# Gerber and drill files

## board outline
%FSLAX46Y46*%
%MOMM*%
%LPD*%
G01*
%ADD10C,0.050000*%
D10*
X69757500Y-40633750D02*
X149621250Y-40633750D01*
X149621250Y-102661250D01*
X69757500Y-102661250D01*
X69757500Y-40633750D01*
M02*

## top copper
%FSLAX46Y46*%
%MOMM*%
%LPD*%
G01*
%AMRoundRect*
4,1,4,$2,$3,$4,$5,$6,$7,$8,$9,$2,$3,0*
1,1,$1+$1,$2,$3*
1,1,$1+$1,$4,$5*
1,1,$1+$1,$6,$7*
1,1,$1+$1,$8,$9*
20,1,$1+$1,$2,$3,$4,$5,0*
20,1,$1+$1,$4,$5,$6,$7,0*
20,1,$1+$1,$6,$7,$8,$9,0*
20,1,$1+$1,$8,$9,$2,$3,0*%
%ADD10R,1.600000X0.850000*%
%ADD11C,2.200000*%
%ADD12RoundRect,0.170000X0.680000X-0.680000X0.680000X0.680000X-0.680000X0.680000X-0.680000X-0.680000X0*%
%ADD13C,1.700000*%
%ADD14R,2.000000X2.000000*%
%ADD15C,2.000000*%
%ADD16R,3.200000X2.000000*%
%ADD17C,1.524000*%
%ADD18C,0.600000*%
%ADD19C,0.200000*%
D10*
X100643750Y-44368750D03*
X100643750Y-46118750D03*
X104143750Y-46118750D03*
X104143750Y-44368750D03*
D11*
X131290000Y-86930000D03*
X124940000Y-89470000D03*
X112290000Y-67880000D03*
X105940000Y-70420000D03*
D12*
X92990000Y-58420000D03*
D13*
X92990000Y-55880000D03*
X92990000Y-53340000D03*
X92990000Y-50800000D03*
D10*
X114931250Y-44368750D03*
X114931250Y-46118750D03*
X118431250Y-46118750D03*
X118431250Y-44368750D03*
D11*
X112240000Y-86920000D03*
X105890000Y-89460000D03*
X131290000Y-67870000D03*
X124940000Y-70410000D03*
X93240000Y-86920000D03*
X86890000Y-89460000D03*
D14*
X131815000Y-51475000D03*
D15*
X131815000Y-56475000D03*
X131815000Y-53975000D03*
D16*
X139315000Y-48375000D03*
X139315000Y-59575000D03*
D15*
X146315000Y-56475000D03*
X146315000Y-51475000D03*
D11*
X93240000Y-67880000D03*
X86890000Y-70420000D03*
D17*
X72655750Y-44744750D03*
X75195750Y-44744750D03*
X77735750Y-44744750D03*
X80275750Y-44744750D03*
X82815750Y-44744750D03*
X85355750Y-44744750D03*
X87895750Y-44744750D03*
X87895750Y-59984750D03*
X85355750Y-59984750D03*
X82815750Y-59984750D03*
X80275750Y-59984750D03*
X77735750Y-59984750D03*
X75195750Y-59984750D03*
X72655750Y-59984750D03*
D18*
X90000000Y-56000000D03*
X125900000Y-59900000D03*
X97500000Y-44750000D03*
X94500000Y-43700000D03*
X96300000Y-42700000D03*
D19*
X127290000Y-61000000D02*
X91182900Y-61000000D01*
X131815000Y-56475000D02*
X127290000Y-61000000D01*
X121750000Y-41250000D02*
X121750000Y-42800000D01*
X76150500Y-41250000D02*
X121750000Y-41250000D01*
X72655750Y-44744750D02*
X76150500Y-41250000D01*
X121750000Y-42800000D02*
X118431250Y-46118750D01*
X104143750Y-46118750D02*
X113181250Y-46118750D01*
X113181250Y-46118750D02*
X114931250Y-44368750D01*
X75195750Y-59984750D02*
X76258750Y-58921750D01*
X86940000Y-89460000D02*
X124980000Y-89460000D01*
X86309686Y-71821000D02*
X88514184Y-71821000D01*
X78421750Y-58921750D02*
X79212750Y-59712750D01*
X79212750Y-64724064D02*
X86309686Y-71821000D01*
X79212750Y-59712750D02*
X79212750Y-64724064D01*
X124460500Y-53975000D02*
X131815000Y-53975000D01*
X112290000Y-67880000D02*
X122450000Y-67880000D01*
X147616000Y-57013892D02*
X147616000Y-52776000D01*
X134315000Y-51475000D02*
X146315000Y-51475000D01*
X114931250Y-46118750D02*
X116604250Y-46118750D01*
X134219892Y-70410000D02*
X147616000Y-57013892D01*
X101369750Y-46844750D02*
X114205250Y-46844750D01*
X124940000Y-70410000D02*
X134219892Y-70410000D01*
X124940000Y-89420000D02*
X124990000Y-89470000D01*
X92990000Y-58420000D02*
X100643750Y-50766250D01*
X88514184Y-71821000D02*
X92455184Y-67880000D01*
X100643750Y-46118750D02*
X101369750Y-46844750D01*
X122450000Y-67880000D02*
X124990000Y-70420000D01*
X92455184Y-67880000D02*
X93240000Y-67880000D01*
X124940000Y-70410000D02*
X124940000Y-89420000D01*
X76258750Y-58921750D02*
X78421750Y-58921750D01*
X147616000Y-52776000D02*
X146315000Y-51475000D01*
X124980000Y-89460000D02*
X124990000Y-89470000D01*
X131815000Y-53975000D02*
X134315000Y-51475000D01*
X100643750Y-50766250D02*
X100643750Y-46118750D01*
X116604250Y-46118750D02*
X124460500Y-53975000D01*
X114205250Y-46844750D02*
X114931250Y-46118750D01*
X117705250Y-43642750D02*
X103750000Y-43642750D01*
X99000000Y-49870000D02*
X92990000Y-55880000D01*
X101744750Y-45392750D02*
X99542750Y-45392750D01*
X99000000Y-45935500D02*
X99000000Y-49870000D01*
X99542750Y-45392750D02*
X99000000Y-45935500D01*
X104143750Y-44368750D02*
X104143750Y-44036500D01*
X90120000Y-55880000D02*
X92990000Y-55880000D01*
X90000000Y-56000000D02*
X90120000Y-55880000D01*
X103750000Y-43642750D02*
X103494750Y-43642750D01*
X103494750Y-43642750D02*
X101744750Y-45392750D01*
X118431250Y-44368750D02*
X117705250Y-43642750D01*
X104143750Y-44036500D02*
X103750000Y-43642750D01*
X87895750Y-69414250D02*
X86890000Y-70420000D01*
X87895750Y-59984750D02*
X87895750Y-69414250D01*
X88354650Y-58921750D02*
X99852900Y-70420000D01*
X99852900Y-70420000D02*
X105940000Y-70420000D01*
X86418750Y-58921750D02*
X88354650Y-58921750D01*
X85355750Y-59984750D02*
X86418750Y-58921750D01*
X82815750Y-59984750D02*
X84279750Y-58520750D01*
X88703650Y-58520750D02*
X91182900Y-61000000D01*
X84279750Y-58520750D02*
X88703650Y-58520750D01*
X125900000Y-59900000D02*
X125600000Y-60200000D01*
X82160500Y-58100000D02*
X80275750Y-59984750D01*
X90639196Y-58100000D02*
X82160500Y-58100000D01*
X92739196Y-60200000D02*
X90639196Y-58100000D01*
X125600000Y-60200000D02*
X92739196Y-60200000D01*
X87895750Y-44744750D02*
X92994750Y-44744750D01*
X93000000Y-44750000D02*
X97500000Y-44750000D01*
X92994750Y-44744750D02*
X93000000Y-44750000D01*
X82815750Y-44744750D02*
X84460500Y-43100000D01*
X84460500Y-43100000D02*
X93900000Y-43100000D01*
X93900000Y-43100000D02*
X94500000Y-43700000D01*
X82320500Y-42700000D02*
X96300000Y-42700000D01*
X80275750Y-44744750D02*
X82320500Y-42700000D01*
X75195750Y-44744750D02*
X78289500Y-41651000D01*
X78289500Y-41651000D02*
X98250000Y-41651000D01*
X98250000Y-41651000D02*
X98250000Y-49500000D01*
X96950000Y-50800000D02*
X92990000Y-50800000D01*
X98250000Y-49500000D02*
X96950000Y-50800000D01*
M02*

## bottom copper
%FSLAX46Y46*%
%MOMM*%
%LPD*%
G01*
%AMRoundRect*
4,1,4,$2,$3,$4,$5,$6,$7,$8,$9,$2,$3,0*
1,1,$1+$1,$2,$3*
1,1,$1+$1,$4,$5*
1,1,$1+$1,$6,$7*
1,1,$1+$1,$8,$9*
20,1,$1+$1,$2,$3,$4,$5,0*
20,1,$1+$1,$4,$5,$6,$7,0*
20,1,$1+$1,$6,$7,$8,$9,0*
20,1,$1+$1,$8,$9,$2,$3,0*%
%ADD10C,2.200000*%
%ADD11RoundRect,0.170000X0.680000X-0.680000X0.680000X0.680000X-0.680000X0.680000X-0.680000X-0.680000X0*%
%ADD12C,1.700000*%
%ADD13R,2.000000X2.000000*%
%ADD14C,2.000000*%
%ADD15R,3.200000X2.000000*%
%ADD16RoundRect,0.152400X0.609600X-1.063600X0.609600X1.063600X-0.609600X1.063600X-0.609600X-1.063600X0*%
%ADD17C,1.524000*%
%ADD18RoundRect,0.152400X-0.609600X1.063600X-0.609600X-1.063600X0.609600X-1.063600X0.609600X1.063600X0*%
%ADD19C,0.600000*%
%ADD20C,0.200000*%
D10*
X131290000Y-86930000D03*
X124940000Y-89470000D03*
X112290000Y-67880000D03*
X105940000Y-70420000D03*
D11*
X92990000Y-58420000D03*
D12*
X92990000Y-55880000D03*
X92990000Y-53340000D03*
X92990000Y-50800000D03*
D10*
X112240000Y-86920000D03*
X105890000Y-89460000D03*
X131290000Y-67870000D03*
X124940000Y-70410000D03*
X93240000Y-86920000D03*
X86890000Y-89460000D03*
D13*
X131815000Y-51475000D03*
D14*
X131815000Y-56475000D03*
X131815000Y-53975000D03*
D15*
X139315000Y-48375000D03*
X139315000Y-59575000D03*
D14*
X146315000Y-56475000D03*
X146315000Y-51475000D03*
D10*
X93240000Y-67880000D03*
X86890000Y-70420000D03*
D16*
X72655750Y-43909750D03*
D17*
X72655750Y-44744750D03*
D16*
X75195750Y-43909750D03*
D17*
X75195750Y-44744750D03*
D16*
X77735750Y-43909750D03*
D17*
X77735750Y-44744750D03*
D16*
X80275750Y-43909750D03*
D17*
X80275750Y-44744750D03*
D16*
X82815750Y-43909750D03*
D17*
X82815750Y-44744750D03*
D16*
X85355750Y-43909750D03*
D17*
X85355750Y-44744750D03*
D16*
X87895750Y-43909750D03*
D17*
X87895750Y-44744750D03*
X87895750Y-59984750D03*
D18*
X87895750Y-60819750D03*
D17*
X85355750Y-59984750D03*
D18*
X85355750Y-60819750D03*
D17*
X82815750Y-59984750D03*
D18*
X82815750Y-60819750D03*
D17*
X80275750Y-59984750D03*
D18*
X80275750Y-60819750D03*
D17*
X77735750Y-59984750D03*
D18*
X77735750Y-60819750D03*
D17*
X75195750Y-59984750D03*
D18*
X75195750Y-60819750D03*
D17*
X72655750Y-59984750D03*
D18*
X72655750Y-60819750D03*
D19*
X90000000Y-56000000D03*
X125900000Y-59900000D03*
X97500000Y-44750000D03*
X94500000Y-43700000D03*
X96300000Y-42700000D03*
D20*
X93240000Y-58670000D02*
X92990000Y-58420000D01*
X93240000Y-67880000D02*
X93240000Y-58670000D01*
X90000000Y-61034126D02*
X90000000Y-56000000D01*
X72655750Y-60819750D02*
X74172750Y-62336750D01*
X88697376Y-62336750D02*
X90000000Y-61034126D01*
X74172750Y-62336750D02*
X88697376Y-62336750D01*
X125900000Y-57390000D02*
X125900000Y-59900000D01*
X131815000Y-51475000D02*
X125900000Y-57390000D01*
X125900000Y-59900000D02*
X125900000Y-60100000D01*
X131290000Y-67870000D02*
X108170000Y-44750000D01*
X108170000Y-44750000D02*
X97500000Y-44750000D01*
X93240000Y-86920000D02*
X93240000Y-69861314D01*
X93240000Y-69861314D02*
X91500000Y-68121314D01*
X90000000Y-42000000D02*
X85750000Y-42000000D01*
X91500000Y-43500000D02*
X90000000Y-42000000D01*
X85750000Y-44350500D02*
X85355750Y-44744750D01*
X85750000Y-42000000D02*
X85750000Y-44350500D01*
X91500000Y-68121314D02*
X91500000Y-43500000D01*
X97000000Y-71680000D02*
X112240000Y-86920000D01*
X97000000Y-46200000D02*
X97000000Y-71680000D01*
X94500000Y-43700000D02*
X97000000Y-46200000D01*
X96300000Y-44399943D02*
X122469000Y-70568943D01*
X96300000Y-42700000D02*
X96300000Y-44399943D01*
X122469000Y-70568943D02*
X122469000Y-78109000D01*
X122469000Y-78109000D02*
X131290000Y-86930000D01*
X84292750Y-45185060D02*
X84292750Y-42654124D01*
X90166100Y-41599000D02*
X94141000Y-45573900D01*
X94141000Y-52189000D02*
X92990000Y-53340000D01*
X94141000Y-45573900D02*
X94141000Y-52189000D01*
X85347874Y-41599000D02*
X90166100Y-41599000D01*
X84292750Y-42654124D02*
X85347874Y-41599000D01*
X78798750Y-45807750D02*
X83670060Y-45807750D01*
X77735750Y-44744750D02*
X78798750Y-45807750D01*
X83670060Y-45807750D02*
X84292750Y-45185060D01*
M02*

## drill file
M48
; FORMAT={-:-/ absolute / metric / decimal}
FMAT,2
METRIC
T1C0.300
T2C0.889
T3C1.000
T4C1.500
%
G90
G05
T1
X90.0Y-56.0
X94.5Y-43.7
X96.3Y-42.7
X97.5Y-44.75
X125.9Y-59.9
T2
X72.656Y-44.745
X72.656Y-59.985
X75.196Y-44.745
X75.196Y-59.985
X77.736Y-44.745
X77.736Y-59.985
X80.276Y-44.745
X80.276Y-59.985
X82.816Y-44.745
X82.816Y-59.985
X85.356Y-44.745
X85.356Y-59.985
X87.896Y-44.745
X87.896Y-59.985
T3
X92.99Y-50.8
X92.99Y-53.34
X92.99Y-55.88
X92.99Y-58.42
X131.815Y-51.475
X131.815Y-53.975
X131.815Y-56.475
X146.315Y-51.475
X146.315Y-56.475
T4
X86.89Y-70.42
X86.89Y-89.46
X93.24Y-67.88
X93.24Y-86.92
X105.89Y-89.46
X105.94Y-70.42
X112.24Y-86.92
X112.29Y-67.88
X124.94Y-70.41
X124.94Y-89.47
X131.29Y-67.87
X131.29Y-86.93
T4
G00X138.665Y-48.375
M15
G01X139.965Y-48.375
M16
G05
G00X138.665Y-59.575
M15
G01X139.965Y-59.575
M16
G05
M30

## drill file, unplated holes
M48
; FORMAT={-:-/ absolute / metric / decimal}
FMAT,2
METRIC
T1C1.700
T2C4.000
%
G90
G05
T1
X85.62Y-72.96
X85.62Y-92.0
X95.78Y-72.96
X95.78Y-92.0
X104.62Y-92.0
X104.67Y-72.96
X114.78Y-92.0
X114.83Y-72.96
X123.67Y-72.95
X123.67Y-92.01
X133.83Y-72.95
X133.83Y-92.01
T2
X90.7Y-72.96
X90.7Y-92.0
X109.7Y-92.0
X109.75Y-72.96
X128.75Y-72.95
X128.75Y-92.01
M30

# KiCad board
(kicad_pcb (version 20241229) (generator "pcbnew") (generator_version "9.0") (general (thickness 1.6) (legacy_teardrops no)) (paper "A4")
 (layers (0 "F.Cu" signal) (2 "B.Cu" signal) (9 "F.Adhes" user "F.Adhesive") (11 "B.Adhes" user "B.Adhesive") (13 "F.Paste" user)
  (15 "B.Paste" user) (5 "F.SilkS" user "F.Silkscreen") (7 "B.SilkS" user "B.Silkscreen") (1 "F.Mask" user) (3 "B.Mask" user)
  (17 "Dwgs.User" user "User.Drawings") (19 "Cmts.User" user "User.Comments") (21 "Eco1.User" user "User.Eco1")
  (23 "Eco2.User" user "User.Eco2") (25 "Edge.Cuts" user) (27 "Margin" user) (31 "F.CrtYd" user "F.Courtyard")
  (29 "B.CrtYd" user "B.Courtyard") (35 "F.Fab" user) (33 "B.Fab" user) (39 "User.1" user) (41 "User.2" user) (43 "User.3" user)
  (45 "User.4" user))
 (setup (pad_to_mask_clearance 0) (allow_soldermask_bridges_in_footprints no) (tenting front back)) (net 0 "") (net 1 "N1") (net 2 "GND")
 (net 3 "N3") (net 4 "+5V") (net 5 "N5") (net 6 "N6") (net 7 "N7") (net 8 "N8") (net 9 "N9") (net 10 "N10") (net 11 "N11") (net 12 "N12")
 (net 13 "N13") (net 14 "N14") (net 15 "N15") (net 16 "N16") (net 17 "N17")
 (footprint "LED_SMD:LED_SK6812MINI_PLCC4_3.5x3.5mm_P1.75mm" (layer "F.Cu") (at 102.39375 45.24375)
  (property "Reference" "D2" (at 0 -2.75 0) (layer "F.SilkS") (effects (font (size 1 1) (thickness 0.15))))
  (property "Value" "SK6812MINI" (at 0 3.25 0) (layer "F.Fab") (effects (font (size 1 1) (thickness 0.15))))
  (pad "1" smd rect (at -1.75 -0.875) (size 1.6 0.85) (layers "F.Cu" "F.Mask" "F.Paste") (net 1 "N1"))
  (pad "2" smd rect (at -1.75 0.875) (size 1.6 0.85) (layers "F.Cu" "F.Mask" "F.Paste") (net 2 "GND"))
  (pad "3" smd rect (at 1.75 0.875) (size 1.6 0.85) (layers "F.Cu" "F.Mask" "F.Paste") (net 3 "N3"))
  (pad "4" smd rect (at 1.75 -0.875) (size 1.6 0.85) (layers "F.Cu" "F.Mask" "F.Paste") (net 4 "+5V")))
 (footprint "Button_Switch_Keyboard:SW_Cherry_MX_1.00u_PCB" (layer "F.Cu") (at 131.29 86.93)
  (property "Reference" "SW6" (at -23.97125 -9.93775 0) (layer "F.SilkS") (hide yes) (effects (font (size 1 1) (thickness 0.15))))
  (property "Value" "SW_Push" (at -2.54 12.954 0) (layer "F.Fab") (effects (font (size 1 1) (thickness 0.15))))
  (pad "" np_thru_hole circle (at -7.62 5.08) (size 1.7 1.7) (drill 1.7) (layers "*.Cu" "*.Mask"))
  (pad "" np_thru_hole circle (at -2.54 5.08) (size 4 4) (drill 4) (layers "*.Cu" "*.Mask"))
  (pad "" np_thru_hole circle (at 2.54 5.08) (size 1.7 1.7) (drill 1.7) (layers "*.Cu" "*.Mask"))
  (pad "1" thru_hole circle (at 0 0) (size 2.2 2.2) (drill 1.5) (layers "*.Cu" "*.Mask") (remove_unused_layers no) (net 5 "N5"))
  (pad "2" thru_hole circle (at -6.35 2.54) (size 2.2 2.2) (drill 1.5) (layers "*.Cu" "*.Mask") (remove_unused_layers no) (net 2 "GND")))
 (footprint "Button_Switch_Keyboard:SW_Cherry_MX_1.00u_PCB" (layer "F.Cu") (at 112.29 67.88)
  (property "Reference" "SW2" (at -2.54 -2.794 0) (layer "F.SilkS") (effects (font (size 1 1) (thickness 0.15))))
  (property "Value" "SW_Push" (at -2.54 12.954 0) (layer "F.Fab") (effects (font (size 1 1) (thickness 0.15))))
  (pad "" np_thru_hole circle (at -7.62 5.08) (size 1.7 1.7) (drill 1.7) (layers "*.Cu" "*.Mask"))
  (pad "" np_thru_hole circle (at -2.54 5.08) (size 4 4) (drill 4) (layers "*.Cu" "*.Mask"))
  (pad "" np_thru_hole circle (at 2.54 5.08) (size 1.7 1.7) (drill 1.7) (layers "*.Cu" "*.Mask"))
  (pad "1" thru_hole circle (at 0 0) (size 2.2 2.2) (drill 1.5) (layers "*.Cu" "*.Mask") (remove_unused_layers no) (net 2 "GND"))
  (pad "2" thru_hole circle (at -6.35 2.54) (size 2.2 2.2) (drill 1.5) (layers "*.Cu" "*.Mask") (remove_unused_layers no) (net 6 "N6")))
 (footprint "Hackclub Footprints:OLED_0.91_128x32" (layer "F.Cu") (at 92.99 58.42 90)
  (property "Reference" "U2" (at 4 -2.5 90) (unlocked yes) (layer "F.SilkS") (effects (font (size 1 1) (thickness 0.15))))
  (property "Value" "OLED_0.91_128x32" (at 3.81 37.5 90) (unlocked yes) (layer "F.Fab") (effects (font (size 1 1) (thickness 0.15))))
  (pad "1" thru_hole roundrect (at 0 0 90) (size 1.7 1.7) (drill 1) (layers "*.Cu" "*.Mask") (remove_unused_layers no)
   (roundrect_rratio 0.1) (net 2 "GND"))
  (pad "2" thru_hole circle (at 2.54 0 90) (size 1.7 1.7) (drill 1) (layers "*.Cu" "*.Mask") (remove_unused_layers no) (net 4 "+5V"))
  (pad "3" thru_hole circle (at 5.08 0 90) (size 1.7 1.7) (drill 1) (layers "*.Cu" "*.Mask") (remove_unused_layers no) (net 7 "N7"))
  (pad "4" thru_hole circle (at 7.62 0 90) (size 1.7 1.7) (drill 1) (layers "*.Cu" "*.Mask") (remove_unused_layers no) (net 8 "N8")))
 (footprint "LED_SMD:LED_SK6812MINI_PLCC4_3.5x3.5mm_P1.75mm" (layer "F.Cu") (at 116.68125 45.24375)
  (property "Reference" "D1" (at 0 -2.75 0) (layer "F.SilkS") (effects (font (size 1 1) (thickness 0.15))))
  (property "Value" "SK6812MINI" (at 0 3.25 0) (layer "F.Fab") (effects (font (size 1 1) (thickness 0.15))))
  (pad "1" smd rect (at -1.75 -0.875) (size 1.6 0.85) (layers "F.Cu" "F.Mask" "F.Paste") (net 3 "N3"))
  (pad "2" smd rect (at -1.75 0.875) (size 1.6 0.85) (layers "F.Cu" "F.Mask" "F.Paste") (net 2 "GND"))
  (pad "3" smd rect (at 1.75 0.875) (size 1.6 0.85) (layers "F.Cu" "F.Mask" "F.Paste") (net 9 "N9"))
  (pad "4" smd rect (at 1.75 -0.875) (size 1.6 0.85) (layers "F.Cu" "F.Mask" "F.Paste") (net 4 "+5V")))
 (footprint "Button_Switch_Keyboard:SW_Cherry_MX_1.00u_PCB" (layer "F.Cu") (at 112.24 86.92)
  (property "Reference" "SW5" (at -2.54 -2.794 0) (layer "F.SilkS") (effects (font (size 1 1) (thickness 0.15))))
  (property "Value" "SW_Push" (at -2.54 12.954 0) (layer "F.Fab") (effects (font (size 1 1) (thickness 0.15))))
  (pad "" np_thru_hole circle (at -7.62 5.08) (size 1.7 1.7) (drill 1.7) (layers "*.Cu" "*.Mask"))
  (pad "" np_thru_hole circle (at -2.54 5.08) (size 4 4) (drill 4) (layers "*.Cu" "*.Mask"))
  (pad "" np_thru_hole circle (at 2.54 5.08) (size 1.7 1.7) (drill 1.7) (layers "*.Cu" "*.Mask"))
  (pad "1" thru_hole circle (at 0 0) (size 2.2 2.2) (drill 1.5) (layers "*.Cu" "*.Mask") (remove_unused_layers no) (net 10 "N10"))
  (pad "2" thru_hole circle (at -6.35 2.54) (size 2.2 2.2) (drill 1.5) (layers "*.Cu" "*.Mask") (remove_unused_layers no) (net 2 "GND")))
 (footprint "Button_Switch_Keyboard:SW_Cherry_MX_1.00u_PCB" (layer "F.Cu") (at 131.29 67.87)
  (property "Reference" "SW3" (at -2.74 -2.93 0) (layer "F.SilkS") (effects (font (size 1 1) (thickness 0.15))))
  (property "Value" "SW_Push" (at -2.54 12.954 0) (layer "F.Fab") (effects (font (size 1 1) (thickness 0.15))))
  (pad "" np_thru_hole circle (at -7.62 5.08) (size 1.7 1.7) (drill 1.7) (layers "*.Cu" "*.Mask"))
  (pad "" np_thru_hole circle (at -2.54 5.08) (size 4 4) (drill 4) (layers "*.Cu" "*.Mask"))
  (pad "" np_thru_hole circle (at 2.54 5.08) (size 1.7 1.7) (drill 1.7) (layers "*.Cu" "*.Mask"))
  (pad "1" thru_hole circle (at 0 0) (size 2.2 2.2) (drill 1.5) (layers "*.Cu" "*.Mask") (remove_unused_layers no) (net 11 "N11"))
  (pad "2" thru_hole circle (at -6.35 2.54) (size 2.2 2.2) (drill 1.5) (layers "*.Cu" "*.Mask") (remove_unused_layers no) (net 2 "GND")))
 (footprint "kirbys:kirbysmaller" (layer "F.Cu") (at 80 51.5)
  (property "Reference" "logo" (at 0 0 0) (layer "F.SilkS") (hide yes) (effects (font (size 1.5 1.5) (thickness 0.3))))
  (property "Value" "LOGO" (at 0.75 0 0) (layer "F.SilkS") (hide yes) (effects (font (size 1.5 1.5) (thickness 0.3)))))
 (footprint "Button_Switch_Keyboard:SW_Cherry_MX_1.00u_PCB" (layer "F.Cu") (at 93.24 86.92)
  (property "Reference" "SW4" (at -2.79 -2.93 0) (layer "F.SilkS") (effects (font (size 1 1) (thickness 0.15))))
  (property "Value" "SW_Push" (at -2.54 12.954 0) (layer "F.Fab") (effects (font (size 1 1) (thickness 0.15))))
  (pad "" np_thru_hole circle (at -7.62 5.08) (size 1.7 1.7) (drill 1.7) (layers "*.Cu" "*.Mask"))
  (pad "" np_thru_hole circle (at -2.54 5.08) (size 4 4) (drill 4) (layers "*.Cu" "*.Mask"))
  (pad "" np_thru_hole circle (at 2.54 5.08) (size 1.7 1.7) (drill 1.7) (layers "*.Cu" "*.Mask"))
  (pad "1" thru_hole circle (at 0 0) (size 2.2 2.2) (drill 1.5) (layers "*.Cu" "*.Mask") (remove_unused_layers no) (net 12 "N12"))
  (pad "2" thru_hole circle (at -6.35 2.54) (size 2.2 2.2) (drill 1.5) (layers "*.Cu" "*.Mask") (remove_unused_layers no) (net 2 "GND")))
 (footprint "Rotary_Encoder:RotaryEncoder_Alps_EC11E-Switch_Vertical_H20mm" (layer "F.Cu") (at 131.815 51.475)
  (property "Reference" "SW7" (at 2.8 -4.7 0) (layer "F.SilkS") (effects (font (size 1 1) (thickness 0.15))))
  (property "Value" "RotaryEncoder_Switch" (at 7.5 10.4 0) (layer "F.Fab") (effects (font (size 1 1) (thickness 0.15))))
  (pad "A" thru_hole rect (at 0 0) (size 2 2) (drill 1) (layers "*.Cu" "*.Mask") (remove_unused_layers no) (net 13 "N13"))
  (pad "B" thru_hole circle (at 0 5) (size 2 2) (drill 1) (layers "*.Cu" "*.Mask") (remove_unused_layers no) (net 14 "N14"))
  (pad "C" thru_hole circle (at 0 2.5) (size 2 2) (drill 1) (layers "*.Cu" "*.Mask") (remove_unused_layers no) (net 2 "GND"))
  (pad "MP" thru_hole rect (at 7.5 -3.1) (size 3.2 2) (drill oval 2.8 1.5) (layers "*.Cu" "*.Mask") (remove_unused_layers no))
  (pad "MP" thru_hole rect (at 7.5 8.1) (size 3.2 2) (drill oval 2.8 1.5) (layers "*.Cu" "*.Mask") (remove_unused_layers no))
  (pad "S1" thru_hole circle (at 14.5 5) (size 2 2) (drill 1) (layers "*.Cu" "*.Mask") (remove_unused_layers no) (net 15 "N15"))
  (pad "S2" thru_hole circle (at 14.5 0) (size 2 2) (drill 1) (layers "*.Cu" "*.Mask") (remove_unused_layers no) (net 2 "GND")))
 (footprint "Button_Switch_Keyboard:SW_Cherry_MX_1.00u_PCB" (layer "F.Cu") (at 93.24 67.88)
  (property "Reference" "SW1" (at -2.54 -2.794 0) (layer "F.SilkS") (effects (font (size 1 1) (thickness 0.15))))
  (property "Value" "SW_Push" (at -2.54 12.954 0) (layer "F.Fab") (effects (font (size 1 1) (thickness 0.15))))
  (pad "" np_thru_hole circle (at -7.62 5.08) (size 1.7 1.7) (drill 1.7) (layers "*.Cu" "*.Mask"))
  (pad "" np_thru_hole circle (at -2.54 5.08) (size 4 4) (drill 4) (layers "*.Cu" "*.Mask"))
  (pad "" np_thru_hole circle (at 2.54 5.08) (size 1.7 1.7) (drill 1.7) (layers "*.Cu" "*.Mask"))
  (pad "1" thru_hole circle (at 0 0) (size 2.2 2.2) (drill 1.5) (layers "*.Cu" "*.Mask") (remove_unused_layers no) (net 2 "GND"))
  (pad "2" thru_hole circle (at -6.35 2.54) (size 2.2 2.2) (drill 1.5) (layers "*.Cu" "*.Mask") (remove_unused_layers no) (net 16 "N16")))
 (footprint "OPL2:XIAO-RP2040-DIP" (layer "B.Cu") (at 80.27575 52.36475 -90)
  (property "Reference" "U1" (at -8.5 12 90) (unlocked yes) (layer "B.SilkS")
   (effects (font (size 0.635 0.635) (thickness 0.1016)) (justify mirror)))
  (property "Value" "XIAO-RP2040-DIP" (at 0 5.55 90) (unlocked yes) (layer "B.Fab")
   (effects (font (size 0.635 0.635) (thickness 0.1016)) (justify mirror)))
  (pad "1" smd roundrect (at -8.455 7.62 90) (size 2.432 1.524) (layers "B.Cu" "B.Mask") (roundrect_rratio 0.1) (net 9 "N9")
   (thermal_bridge_angle 45))
  (pad "1" thru_hole circle (at -7.62 7.62 90) (size 1.524 1.524) (drill 0.889) (layers "*.Cu" "*.Mask") (remove_unused_layers no)
   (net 9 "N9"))
  (pad "2" smd roundrect (at -8.455 5.08 90) (size 2.432 1.524) (layers "B.Cu" "B.Mask") (roundrect_rratio 0.1) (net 8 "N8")
   (thermal_bridge_angle 45))
  (pad "2" thru_hole circle (at -7.62 5.08 90) (size 1.524 1.524) (drill 0.889) (layers "*.Cu" "*.Mask") (remove_unused_layers no)
   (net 8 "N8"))
  (pad "3" smd roundrect (at -8.455 2.54 90) (size 2.432 1.524) (layers "B.Cu" "B.Mask") (roundrect_rratio 0.1) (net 7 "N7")
   (thermal_bridge_angle 45))
  (pad "3" thru_hole circle (at -7.62 2.54 90) (size 1.524 1.524) (drill 0.889) (layers "*.Cu" "*.Mask") (remove_unused_layers no)
   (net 7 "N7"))
  (pad "4" smd roundrect (at -8.455 0 90) (size 2.432 1.524) (layers "B.Cu" "B.Mask") (roundrect_rratio 0.1) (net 5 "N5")
   (thermal_bridge_angle 45))
  (pad "4" thru_hole circle (at -7.62 0 90) (size 1.524 1.524) (drill 0.889) (layers "*.Cu" "*.Mask") (remove_unused_layers no) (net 5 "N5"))
  (pad "5" smd roundrect (at -8.455 -2.54 90) (size 2.432 1.524) (layers "B.Cu" "B.Mask") (roundrect_rratio 0.1) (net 10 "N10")
   (thermal_bridge_angle 45))
  (pad "5" thru_hole circle (at -7.62 -2.54 90) (size 1.524 1.524) (drill 0.889) (layers "*.Cu" "*.Mask") (remove_unused_layers no)
   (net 10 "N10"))
  (pad "6" smd roundrect (at -8.455 -5.08 90) (size 2.432 1.524) (layers "B.Cu" "B.Mask") (roundrect_rratio 0.1) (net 12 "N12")
   (thermal_bridge_angle 45))
  (pad "6" thru_hole circle (at -7.62 -5.08 90) (size 1.524 1.524) (drill 0.889) (layers "*.Cu" "*.Mask") (remove_unused_layers no)
   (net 12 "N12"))
  (pad "7" smd roundrect (at -8.455 -7.62 90) (size 2.432 1.524) (layers "B.Cu" "B.Mask") (roundrect_rratio 0.1) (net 11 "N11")
   (thermal_bridge_angle 45))
  (pad "7" thru_hole circle (at -7.62 -7.62 90) (size 1.524 1.524) (drill 0.889) (layers "*.Cu" "*.Mask") (remove_unused_layers no)
   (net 11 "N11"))
  (pad "8" thru_hole circle (at 7.62 -7.62 270) (size 1.524 1.524) (drill 0.889) (layers "*.Cu" "*.Mask") (remove_unused_layers no)
   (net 16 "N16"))
  (pad "8" smd roundrect (at 8.455 -7.62 270) (size 2.432 1.524) (layers "B.Cu" "B.Mask") (roundrect_rratio 0.1) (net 16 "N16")
   (thermal_bridge_angle 45))
  (pad "9" thru_hole circle (at 7.62 -5.08 270) (size 1.524 1.524) (drill 0.889) (layers "*.Cu" "*.Mask") (remove_unused_layers no)
   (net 6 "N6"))
  (pad "9" smd roundrect (at 8.455 -5.08 270) (size 2.432 1.524) (layers "B.Cu" "B.Mask") (roundrect_rratio 0.1) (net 6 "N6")
   (thermal_bridge_angle 45))
  (pad "10" thru_hole circle (at 7.62 -2.54 270) (size 1.524 1.524) (drill 0.889) (layers "*.Cu" "*.Mask") (remove_unused_layers no)
   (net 14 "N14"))
  (pad "10" smd roundrect (at 8.455 -2.54 270) (size 2.432 1.524) (layers "B.Cu" "B.Mask") (roundrect_rratio 0.1) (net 14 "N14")
   (thermal_bridge_angle 45))
  (pad "11" thru_hole circle (at 7.62 0 270) (size 1.524 1.524) (drill 0.889) (layers "*.Cu" "*.Mask") (remove_unused_layers no)
   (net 13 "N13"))
  (pad "11" smd roundrect (at 8.455 0 270) (size 2.432 1.524) (layers "B.Cu" "B.Mask") (roundrect_rratio 0.1) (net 13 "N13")
   (thermal_bridge_angle 45))
  (pad "12" thru_hole circle (at 7.62 2.54 270) (size 1.524 1.524) (drill 0.889) (layers "*.Cu" "*.Mask") (remove_unused_layers no)
   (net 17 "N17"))
  (pad "12" smd roundrect (at 8.455 2.54 270) (size 2.432 1.524) (layers "B.Cu" "B.Mask") (roundrect_rratio 0.1) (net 17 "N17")
   (thermal_bridge_angle 45))
  (pad "13" thru_hole circle (at 7.62 5.08 270) (size 1.524 1.524) (drill 0.889) (layers "*.Cu" "*.Mask") (remove_unused_layers no)
   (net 2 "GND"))
  (pad "13" smd roundrect (at 8.455 5.08 270) (size 2.432 1.524) (layers "B.Cu" "B.Mask") (roundrect_rratio 0.1) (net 2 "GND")
   (thermal_bridge_angle 45))
  (pad "14" thru_hole circle (at 7.62 7.62 270) (size 1.524 1.524) (drill 0.889) (layers "*.Cu" "*.Mask") (remove_unused_layers no)
   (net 4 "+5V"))
  (pad "14" smd roundrect (at 8.455 7.62 270) (size 2.432 1.524) (layers "B.Cu" "B.Mask") (roundrect_rratio 0.1) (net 4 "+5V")
   (thermal_bridge_angle 45)))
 (gr_rect (start 69.7575 40.63375) (end 149.62125 102.66125) (stroke (width 0.05) (type default)) (fill no) (layer "Edge.Cuts"))
 (segment (start 121.75 41.25) (end 121.75 42.8) (width 0.2) (layer "F.Cu") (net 9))
 (segment (start 76.1505 41.25) (end 121.75 41.25) (width 0.2) (layer "F.Cu") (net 9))
 (segment (start 72.65575 44.74475) (end 76.1505 41.25) (width 0.2) (layer "F.Cu") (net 9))
 (segment (start 121.75 42.8) (end 118.43125 46.11875) (width 0.2) (layer "F.Cu") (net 9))
 (segment (start 104.14375 46.11875) (end 113.18125 46.11875) (width 0.2) (layer "F.Cu") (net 3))
 (segment (start 113.18125 46.11875) (end 114.93125 44.36875) (width 0.2) (layer "F.Cu") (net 3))
 (segment (start 75.19575 59.98475) (end 76.25875 58.92175) (width 0.2) (layer "F.Cu") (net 2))
 (segment (start 86.94 89.46) (end 124.98 89.46) (width 0.2) (layer "F.Cu") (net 2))
 (segment (start 86.309686 71.821) (end 88.514184 71.821) (width 0.2) (layer "F.Cu") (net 2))
 (segment (start 78.42175 58.92175) (end 79.21275 59.71275) (width 0.2) (layer "F.Cu") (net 2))
 (segment (start 79.21275 64.724064) (end 86.309686 71.821) (width 0.2) (layer "F.Cu") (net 2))
 (segment (start 79.21275 59.71275) (end 79.21275 64.724064) (width 0.2) (layer "F.Cu") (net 2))
 (segment (start 124.4605 53.975) (end 131.815 53.975) (width 0.2) (layer "F.Cu") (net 2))
 (segment (start 112.29 67.88) (end 122.45 67.88) (width 0.2) (layer "F.Cu") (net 2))
 (segment (start 147.616 57.013892) (end 147.616 52.776) (width 0.2) (layer "F.Cu") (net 2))
 (segment (start 134.315 51.475) (end 146.315 51.475) (width 0.2) (layer "F.Cu") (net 2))
 (segment (start 114.93125 46.11875) (end 116.60425 46.11875) (width 0.2) (layer "F.Cu") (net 2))
 (segment (start 134.219892 70.41) (end 147.616 57.013892) (width 0.2) (layer "F.Cu") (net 2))
 (segment (start 101.36975 46.84475) (end 114.20525 46.84475) (width 0.2) (layer "F.Cu") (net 2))
 (segment (start 124.94 70.41) (end 134.219892 70.41) (width 0.2) (layer "F.Cu") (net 2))
 (segment (start 124.94 89.42) (end 124.99 89.47) (width 0.2) (layer "F.Cu") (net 2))
 (segment (start 92.99 58.42) (end 100.64375 50.76625) (width 0.2) (layer "F.Cu") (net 2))
 (segment (start 88.514184 71.821) (end 92.455184 67.88) (width 0.2) (layer "F.Cu") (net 2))
 (segment (start 100.64375 46.11875) (end 101.36975 46.84475) (width 0.2) (layer "F.Cu") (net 2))
 (segment (start 122.45 67.88) (end 124.99 70.42) (width 0.2) (layer "F.Cu") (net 2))
 (segment (start 92.455184 67.88) (end 93.24 67.88) (width 0.2) (layer "F.Cu") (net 2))
 (segment (start 124.94 70.41) (end 124.94 89.42) (width 0.2) (layer "F.Cu") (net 2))
 (segment (start 76.25875 58.92175) (end 78.42175 58.92175) (width 0.2) (layer "F.Cu") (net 2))
 (segment (start 147.616 52.776) (end 146.315 51.475) (width 0.2) (layer "F.Cu") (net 2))
 (segment (start 124.98 89.46) (end 124.99 89.47) (width 0.2) (layer "F.Cu") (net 2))
 (segment (start 131.815 53.975) (end 134.315 51.475) (width 0.2) (layer "F.Cu") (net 2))
 (segment (start 100.64375 50.76625) (end 100.64375 46.11875) (width 0.2) (layer "F.Cu") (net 2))
 (segment (start 116.60425 46.11875) (end 124.4605 53.975) (width 0.2) (layer "F.Cu") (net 2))
 (segment (start 114.20525 46.84475) (end 114.93125 46.11875) (width 0.2) (layer "F.Cu") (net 2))
 (segment (start 93.24 58.67) (end 92.99 58.42) (width 0.2) (layer "B.Cu") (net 2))
 (segment (start 93.24 67.88) (end 93.24 58.67) (width 0.2) (layer "B.Cu") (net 2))
 (segment (start 117.70525 43.64275) (end 103.75 43.64275) (width 0.2) (layer "F.Cu") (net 4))
 (segment (start 99 49.87) (end 92.99 55.88) (width 0.2) (layer "F.Cu") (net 4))
 (segment (start 101.74475 45.39275) (end 99.54275 45.39275) (width 0.2) (layer "F.Cu") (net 4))
 (segment (start 99 45.9355) (end 99 49.87) (width 0.2) (layer "F.Cu") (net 4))
 (segment (start 99.54275 45.39275) (end 99 45.9355) (width 0.2) (layer "F.Cu") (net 4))
 (segment (start 104.14375 44.36875) (end 104.14375 44.0365) (width 0.2) (layer "F.Cu") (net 4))
 (segment (start 90.12 55.88) (end 92.99 55.88) (width 0.2) (layer "F.Cu") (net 4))
 (segment (start 90 56) (end 90.12 55.88) (width 0.2) (layer "F.Cu") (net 4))
 (segment (start 103.75 43.64275) (end 103.49475 43.64275) (width 0.2) (layer "F.Cu") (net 4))
 (segment (start 103.49475 43.64275) (end 101.74475 45.39275) (width 0.2) (layer "F.Cu") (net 4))
 (segment (start 118.43125 44.36875) (end 117.70525 43.64275) (width 0.2) (layer "F.Cu") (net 4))
 (segment (start 104.14375 44.0365) (end 103.75 43.64275) (width 0.2) (layer "F.Cu") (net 4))
 (via (at 90 56) (size 0.6) (drill 0.3) (layers "F.Cu" "B.Cu") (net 4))
 (segment (start 90 61.034126) (end 90 56) (width 0.2) (layer "B.Cu") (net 4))
 (segment (start 72.65575 60.81975) (end 74.17275 62.33675) (width 0.2) (layer "B.Cu") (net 4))
 (segment (start 88.697376 62.33675) (end 90 61.034126) (width 0.2) (layer "B.Cu") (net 4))
 (segment (start 74.17275 62.33675) (end 88.697376 62.33675) (width 0.2) (layer "B.Cu") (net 4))
 (segment (start 87.89575 69.41425) (end 86.89 70.42) (width 0.2) (layer "F.Cu") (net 16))
 (segment (start 87.89575 59.98475) (end 87.89575 69.41425) (width 0.2) (layer "F.Cu") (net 16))
 (segment (start 88.35465 58.92175) (end 99.8529 70.42) (width 0.2) (layer "F.Cu") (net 6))
 (segment (start 99.8529 70.42) (end 105.94 70.42) (width 0.2) (layer "F.Cu") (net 6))
 (segment (start 86.41875 58.92175) (end 88.35465 58.92175) (width 0.2) (layer "F.Cu") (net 6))
 (segment (start 85.35575 59.98475) (end 86.41875 58.92175) (width 0.2) (layer "F.Cu") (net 6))
 (segment (start 82.81575 59.98475) (end 84.27975 58.52075) (width 0.2) (layer "F.Cu") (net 14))
 (segment (start 127.29 61) (end 91.1829 61) (width 0.2) (layer "F.Cu") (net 14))
 (segment (start 88.70365 58.52075) (end 91.1829 61) (width 0.2) (layer "F.Cu") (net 14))
 (segment (start 131.815 56.475) (end 127.29 61) (width 0.2) (layer "F.Cu") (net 14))
 (segment (start 84.27975 58.52075) (end 88.70365 58.52075) (width 0.2) (layer "F.Cu") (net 14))
 (segment (start 125.9 59.9) (end 125.6 60.2) (width 0.2) (layer "F.Cu") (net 13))
 (segment (start 82.1605 58.1) (end 80.27575 59.98475) (width 0.2) (layer "F.Cu") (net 13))
 (segment (start 90.639196 58.1) (end 82.1605 58.1) (width 0.2) (layer "F.Cu") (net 13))
 (segment (start 92.739196 60.2) (end 90.639196 58.1) (width 0.2) (layer "F.Cu") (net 13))
 (segment (start 125.6 60.2) (end 92.739196 60.2) (width 0.2) (layer "F.Cu") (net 13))
 (via (at 125.9 59.9) (size 0.6) (drill 0.3) (layers "F.Cu" "B.Cu") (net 13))
 (segment (start 125.9 57.39) (end 125.9 59.9) (width 0.2) (layer "B.Cu") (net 13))
 (segment (start 131.815 51.475) (end 125.9 57.39) (width 0.2) (layer "B.Cu") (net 13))
 (segment (start 125.9 59.9) (end 125.9 60.1) (width 0.2) (layer "B.Cu") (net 13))
 (segment (start 87.89575 44.74475) (end 92.99475 44.74475) (width 0.2) (layer "F.Cu") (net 11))
 (segment (start 93 44.75) (end 97.5 44.75) (width 0.2) (layer "F.Cu") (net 11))
 (segment (start 92.99475 44.74475) (end 93 44.75) (width 0.2) (layer "F.Cu") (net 11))
 (via (at 97.5 44.75) (size 0.6) (drill 0.3) (layers "F.Cu" "B.Cu") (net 11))
 (segment (start 131.29 67.87) (end 108.17 44.75) (width 0.2) (layer "B.Cu") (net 11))
 (segment (start 108.17 44.75) (end 97.5 44.75) (width 0.2) (layer "B.Cu") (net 11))
 (segment (start 93.24 86.92) (end 93.24 69.861314) (width 0.2) (layer "B.Cu") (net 12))
 (segment (start 93.24 69.861314) (end 91.5 68.121314) (width 0.2) (layer "B.Cu") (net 12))
 (segment (start 90 42) (end 85.75 42) (width 0.2) (layer "B.Cu") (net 12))
 (segment (start 91.5 43.5) (end 90 42) (width 0.2) (layer "B.Cu") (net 12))
 (segment (start 85.75 44.3505) (end 85.35575 44.74475) (width 0.2) (layer "B.Cu") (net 12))
 (segment (start 85.75 42) (end 85.75 44.3505) (width 0.2) (layer "B.Cu") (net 12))
 (segment (start 91.5 68.121314) (end 91.5 43.5) (width 0.2) (layer "B.Cu") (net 12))
 (segment (start 82.81575 44.74475) (end 84.4605 43.1) (width 0.2) (layer "F.Cu") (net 10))
 (segment (start 84.4605 43.1) (end 93.9 43.1) (width 0.2) (layer "F.Cu") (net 10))
 (segment (start 93.9 43.1) (end 94.5 43.7) (width 0.2) (layer "F.Cu") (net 10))
 (via (at 94.5 43.7) (size 0.6) (drill 0.3) (layers "F.Cu" "B.Cu") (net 10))
 (segment (start 97 71.68) (end 112.24 86.92) (width 0.2) (layer "B.Cu") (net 10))
 (segment (start 97 46.2) (end 97 71.68) (width 0.2) (layer "B.Cu") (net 10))
 (segment (start 94.5 43.7) (end 97 46.2) (width 0.2) (layer "B.Cu") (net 10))
 (segment (start 82.3205 42.7) (end 96.3 42.7) (width 0.2) (layer "F.Cu") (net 5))
 (segment (start 80.27575 44.74475) (end 82.3205 42.7) (width 0.2) (layer "F.Cu") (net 5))
 (via (at 96.3 42.7) (size 0.6) (drill 0.3) (layers "F.Cu" "B.Cu") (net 5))
 (segment (start 96.3 44.399943) (end 122.469 70.568943) (width 0.2) (layer "B.Cu") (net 5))
 (segment (start 96.3 42.7) (end 96.3 44.399943) (width 0.2) (layer "B.Cu") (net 5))
 (segment (start 122.469 70.568943) (end 122.469 78.109) (width 0.2) (layer "B.Cu") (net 5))
 (segment (start 122.469 78.109) (end 131.29 86.93) (width 0.2) (layer "B.Cu") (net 5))
 (segment (start 84.29275 45.18506) (end 84.29275 42.654124) (width 0.2) (layer "B.Cu") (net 7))
 (segment (start 90.1661 41.599) (end 94.141 45.5739) (width 0.2) (layer "B.Cu") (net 7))
 (segment (start 94.141 52.189) (end 92.99 53.34) (width 0.2) (layer "B.Cu") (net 7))
 (segment (start 94.141 45.5739) (end 94.141 52.189) (width 0.2) (layer "B.Cu") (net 7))
 (segment (start 85.347874 41.599) (end 90.1661 41.599) (width 0.2) (layer "B.Cu") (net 7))
 (segment (start 84.29275 42.654124) (end 85.347874 41.599) (width 0.2) (layer "B.Cu") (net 7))
 (segment (start 78.79875 45.80775) (end 83.67006 45.80775) (width 0.2) (layer "B.Cu") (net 7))
 (segment (start 77.73575 44.74475) (end 78.79875 45.80775) (width 0.2) (layer "B.Cu") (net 7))
 (segment (start 83.67006 45.80775) (end 84.29275 45.18506) (width 0.2) (layer "B.Cu") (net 7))
 (segment (start 75.19575 44.74475) (end 78.2895 41.651) (width 0.2) (layer "F.Cu") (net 8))
 (segment (start 78.2895 41.651) (end 98.25 41.651) (width 0.2) (layer "F.Cu") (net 8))
 (segment (start 98.25 41.651) (end 98.25 49.5) (width 0.2) (layer "F.Cu") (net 8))
 (segment (start 96.95 50.8) (end 92.99 50.8) (width 0.2) (layer "F.Cu") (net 8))
 (segment (start 98.25 49.5) (end 96.95 50.8) (width 0.2) (layer "F.Cu") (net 8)))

